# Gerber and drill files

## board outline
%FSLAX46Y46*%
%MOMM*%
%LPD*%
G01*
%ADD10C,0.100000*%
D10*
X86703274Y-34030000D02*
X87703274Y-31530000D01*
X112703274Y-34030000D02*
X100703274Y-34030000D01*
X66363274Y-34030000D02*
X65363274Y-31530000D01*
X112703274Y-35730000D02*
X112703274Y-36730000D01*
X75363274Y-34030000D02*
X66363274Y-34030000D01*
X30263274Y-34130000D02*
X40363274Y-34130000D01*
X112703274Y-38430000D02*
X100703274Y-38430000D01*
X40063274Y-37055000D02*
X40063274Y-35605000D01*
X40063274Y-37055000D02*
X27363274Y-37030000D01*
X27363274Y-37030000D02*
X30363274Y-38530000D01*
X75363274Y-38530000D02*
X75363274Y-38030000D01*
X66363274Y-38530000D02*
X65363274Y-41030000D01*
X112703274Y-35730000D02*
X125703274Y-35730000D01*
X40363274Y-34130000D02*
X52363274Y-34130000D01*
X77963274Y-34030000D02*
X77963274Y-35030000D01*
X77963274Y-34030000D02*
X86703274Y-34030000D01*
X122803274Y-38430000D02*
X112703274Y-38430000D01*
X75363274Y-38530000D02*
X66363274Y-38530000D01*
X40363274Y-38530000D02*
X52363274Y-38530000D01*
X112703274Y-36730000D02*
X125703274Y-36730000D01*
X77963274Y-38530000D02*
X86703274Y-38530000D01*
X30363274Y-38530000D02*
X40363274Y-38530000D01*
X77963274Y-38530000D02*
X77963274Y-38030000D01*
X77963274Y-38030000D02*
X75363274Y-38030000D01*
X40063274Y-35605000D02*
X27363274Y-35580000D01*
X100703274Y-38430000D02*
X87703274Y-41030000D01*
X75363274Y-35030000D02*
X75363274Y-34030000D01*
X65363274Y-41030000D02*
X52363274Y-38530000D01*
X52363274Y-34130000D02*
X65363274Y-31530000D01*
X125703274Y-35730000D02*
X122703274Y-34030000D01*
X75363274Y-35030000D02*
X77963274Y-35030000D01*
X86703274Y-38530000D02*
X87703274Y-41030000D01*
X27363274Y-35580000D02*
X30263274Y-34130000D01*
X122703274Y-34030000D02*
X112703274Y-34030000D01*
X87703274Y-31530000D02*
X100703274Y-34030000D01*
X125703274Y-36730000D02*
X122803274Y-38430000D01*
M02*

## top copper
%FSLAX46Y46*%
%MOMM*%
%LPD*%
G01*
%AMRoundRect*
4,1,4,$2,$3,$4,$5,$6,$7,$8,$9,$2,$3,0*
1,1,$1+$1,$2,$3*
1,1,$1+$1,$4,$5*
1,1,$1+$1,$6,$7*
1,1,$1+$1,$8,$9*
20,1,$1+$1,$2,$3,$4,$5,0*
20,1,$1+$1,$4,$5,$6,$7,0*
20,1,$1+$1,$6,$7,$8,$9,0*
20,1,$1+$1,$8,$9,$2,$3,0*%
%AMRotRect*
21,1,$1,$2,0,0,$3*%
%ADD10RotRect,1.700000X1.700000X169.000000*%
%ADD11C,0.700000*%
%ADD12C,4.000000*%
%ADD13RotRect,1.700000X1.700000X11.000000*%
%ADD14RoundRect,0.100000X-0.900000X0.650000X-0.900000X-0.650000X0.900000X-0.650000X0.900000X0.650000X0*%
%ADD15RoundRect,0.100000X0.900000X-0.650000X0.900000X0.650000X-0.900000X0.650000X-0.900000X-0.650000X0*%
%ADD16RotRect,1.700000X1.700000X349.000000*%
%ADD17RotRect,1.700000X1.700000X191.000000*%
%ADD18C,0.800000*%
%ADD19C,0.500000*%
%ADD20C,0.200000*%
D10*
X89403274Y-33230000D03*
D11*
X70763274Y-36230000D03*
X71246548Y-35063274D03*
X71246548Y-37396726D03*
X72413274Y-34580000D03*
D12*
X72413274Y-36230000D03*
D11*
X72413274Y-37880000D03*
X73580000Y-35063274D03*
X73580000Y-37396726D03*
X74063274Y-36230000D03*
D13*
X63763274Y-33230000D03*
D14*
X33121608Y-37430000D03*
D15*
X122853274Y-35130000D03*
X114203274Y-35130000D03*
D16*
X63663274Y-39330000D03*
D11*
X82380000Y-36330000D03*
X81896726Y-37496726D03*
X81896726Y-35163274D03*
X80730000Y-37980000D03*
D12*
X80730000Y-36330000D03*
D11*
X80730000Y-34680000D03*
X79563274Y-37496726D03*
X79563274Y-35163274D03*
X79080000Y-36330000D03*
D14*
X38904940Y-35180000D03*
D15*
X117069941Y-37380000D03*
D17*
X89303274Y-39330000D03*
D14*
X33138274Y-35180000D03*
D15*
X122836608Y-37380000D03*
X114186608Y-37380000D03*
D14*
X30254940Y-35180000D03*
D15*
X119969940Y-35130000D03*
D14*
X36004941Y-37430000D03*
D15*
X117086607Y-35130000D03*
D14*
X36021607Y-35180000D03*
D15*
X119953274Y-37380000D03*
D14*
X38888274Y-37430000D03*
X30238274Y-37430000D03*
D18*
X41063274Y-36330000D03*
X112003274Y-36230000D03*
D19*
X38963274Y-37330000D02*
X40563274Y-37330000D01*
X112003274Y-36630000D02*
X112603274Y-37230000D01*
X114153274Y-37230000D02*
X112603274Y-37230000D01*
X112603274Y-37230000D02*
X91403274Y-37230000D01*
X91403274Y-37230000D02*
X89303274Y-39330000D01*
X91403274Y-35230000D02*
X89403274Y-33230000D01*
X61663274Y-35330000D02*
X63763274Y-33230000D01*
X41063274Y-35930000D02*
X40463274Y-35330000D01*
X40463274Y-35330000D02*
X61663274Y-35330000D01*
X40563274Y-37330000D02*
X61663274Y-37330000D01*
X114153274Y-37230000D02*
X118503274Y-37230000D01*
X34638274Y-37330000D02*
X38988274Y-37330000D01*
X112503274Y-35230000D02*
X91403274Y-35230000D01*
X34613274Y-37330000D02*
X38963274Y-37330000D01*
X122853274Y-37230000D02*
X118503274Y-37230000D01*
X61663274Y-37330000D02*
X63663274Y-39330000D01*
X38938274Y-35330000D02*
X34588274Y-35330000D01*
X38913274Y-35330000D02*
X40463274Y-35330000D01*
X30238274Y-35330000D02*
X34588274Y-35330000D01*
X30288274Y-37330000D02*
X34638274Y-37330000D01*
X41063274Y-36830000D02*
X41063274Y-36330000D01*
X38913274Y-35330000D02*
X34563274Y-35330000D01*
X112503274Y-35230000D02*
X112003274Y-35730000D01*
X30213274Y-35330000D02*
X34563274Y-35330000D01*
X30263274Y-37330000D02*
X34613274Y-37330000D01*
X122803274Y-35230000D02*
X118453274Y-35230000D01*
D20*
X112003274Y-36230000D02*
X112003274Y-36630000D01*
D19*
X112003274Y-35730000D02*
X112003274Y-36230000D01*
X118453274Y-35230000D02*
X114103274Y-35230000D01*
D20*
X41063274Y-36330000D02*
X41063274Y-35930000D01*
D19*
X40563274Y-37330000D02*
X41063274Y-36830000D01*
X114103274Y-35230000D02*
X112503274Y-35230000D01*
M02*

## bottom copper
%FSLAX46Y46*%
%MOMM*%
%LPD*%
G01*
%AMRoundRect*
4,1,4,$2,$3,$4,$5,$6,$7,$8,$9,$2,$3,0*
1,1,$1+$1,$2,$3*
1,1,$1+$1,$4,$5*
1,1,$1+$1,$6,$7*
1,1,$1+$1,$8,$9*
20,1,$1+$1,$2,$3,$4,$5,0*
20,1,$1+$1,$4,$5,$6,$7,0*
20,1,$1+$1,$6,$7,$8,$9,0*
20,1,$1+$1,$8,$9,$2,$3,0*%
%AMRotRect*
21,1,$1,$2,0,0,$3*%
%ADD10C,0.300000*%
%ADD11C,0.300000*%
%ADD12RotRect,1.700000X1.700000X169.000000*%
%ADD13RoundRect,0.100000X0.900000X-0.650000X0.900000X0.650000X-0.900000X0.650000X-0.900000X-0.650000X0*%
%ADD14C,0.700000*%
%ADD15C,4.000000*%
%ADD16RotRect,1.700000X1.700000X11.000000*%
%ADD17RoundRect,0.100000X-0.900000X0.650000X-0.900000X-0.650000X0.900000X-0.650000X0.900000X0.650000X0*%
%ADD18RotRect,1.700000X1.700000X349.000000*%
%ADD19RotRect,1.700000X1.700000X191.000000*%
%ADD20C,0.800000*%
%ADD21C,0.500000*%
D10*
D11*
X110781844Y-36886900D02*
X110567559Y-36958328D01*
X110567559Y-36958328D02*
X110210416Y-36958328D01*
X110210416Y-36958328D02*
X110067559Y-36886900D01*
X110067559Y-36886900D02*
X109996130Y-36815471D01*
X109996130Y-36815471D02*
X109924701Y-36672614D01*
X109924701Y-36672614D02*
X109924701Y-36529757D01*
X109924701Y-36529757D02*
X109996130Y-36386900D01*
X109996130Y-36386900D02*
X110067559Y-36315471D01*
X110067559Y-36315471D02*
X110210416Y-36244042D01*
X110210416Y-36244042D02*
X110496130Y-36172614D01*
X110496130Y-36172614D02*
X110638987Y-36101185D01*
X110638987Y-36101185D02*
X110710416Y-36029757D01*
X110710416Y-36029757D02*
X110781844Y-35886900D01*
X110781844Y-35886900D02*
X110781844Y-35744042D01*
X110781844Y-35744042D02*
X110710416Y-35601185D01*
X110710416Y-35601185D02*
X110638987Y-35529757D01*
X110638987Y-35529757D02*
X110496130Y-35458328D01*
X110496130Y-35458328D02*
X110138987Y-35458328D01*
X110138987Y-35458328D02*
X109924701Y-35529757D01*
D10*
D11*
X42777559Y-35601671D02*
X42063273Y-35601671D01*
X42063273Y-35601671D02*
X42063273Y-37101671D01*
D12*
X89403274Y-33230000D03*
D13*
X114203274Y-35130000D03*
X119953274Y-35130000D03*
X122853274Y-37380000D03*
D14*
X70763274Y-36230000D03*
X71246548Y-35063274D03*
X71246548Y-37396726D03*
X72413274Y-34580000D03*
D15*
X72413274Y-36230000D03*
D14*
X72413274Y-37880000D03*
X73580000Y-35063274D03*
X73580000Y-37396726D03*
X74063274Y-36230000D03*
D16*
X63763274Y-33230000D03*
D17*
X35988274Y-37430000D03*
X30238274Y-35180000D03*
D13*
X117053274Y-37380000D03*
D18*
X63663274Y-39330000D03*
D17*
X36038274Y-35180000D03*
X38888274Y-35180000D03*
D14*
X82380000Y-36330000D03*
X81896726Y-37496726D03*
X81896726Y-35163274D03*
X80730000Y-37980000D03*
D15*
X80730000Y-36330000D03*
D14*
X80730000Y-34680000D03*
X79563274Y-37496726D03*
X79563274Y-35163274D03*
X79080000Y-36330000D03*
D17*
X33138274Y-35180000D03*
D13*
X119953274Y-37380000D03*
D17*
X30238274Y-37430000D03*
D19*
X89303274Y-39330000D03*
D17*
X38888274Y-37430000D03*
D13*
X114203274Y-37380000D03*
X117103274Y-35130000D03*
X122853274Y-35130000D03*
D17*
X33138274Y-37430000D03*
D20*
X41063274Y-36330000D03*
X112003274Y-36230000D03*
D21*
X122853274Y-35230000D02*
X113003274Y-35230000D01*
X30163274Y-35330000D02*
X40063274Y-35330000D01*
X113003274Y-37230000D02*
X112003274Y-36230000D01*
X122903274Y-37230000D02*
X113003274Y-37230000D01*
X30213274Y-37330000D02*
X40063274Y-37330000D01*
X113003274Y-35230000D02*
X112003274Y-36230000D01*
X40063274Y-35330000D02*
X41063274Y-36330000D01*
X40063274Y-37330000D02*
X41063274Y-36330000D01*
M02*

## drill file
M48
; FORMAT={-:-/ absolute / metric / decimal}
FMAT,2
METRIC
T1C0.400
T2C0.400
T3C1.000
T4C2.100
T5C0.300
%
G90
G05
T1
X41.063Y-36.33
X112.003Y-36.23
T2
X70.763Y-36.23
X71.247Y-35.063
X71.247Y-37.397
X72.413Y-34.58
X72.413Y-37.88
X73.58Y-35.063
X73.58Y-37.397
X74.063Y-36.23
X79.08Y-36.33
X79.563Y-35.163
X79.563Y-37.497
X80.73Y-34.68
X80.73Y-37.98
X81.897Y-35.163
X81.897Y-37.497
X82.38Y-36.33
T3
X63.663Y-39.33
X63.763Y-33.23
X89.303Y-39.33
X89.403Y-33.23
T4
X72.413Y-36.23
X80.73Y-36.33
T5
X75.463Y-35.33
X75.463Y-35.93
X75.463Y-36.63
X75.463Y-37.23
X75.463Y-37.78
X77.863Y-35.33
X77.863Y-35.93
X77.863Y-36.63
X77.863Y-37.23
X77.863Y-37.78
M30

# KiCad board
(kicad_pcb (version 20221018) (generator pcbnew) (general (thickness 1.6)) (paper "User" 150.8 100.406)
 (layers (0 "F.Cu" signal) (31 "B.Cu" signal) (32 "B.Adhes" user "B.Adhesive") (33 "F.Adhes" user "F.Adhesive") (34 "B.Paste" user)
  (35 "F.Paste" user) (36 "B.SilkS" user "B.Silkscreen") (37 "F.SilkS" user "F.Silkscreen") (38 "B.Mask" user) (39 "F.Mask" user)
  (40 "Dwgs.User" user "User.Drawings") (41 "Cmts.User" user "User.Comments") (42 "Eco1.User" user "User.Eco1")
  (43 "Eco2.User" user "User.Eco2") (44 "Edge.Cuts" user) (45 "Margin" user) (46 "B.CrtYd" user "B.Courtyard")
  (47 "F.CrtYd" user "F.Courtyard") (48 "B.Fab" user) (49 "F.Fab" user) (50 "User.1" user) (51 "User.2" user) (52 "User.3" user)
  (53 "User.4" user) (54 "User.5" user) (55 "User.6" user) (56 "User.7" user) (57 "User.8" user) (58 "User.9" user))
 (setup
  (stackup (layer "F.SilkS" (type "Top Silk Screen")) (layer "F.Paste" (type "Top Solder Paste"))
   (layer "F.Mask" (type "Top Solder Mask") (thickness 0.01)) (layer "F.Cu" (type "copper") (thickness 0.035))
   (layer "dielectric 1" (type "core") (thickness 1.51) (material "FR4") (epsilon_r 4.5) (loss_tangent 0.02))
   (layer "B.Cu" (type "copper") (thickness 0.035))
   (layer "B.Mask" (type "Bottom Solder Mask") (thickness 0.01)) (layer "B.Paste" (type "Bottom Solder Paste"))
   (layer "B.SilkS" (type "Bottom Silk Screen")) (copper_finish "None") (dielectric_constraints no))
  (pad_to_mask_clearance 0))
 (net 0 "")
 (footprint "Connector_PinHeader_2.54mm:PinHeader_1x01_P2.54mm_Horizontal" (layer "F.Cu") (at 89.403274 33.23 169)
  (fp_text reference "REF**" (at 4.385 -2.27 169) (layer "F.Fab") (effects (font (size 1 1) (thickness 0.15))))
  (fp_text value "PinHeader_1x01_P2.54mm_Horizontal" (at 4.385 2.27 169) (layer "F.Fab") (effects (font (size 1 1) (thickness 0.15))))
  (pad "1" thru_hole rect (at 0 0 169) (size 1.7 1.7) (drill 1) (layers "F&B.Cu" "*.Mask")))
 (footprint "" (layer "F.Cu") (at 114.203274 35.13)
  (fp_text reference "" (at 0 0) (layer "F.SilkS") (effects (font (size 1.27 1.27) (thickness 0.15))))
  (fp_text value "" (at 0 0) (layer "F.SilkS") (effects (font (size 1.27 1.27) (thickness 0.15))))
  (pad "2" smd roundrect (at 0 0 90) (size 1.5 2) (layers "B.Cu" "B.Paste" "B.Mask") (roundrect_rratio 0.06666666667)))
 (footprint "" (layer "F.Cu") (at 119.953274 35.13)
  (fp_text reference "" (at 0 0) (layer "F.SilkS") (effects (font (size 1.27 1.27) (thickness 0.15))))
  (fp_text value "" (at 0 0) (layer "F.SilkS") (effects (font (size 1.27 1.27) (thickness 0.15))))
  (pad "2" smd roundrect (at 0 0 90) (size 1.5 2) (layers "B.Cu" "B.Paste" "B.Mask") (roundrect_rratio 0.06666666667)))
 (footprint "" (layer "F.Cu") (at 122.853274 37.38)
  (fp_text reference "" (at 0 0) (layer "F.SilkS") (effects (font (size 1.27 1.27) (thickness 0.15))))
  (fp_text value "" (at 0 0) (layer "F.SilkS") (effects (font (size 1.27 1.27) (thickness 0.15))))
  (pad "2" smd roundrect (at 0 0 90) (size 1.5 2) (layers "B.Cu" "B.Paste" "B.Mask") (roundrect_rratio 0.06666666667)))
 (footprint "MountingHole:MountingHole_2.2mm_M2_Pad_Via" (layer "F.Cu") (at 72.413274 36.23)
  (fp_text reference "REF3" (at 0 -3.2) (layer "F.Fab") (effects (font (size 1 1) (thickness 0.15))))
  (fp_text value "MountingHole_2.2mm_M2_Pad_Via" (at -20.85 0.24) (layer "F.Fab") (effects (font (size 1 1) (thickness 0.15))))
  (pad "1" thru_hole circle (at -1.65 0) (size 0.7 0.7) (drill 0.4) (layers "F&B.Cu" "*.Mask"))
  (pad "1" thru_hole circle (at -1.166726 -1.166726) (size 0.7 0.7) (drill 0.4) (layers "F&B.Cu" "*.Mask"))
  (pad "1" thru_hole circle (at -1.166726 1.166726) (size 0.7 0.7) (drill 0.4) (layers "F&B.Cu" "*.Mask"))
  (pad "1" thru_hole circle (at 0 -1.65) (size 0.7 0.7) (drill 0.4) (layers "F&B.Cu" "*.Mask"))
  (pad "1" thru_hole circle (at 0 0) (size 4 4) (drill 2.1) (layers "F&B.Cu" "*.Mask"))
  (pad "1" thru_hole circle (at 0 1.65) (size 0.7 0.7) (drill 0.4) (layers "F&B.Cu" "*.Mask"))
  (pad "1" thru_hole circle (at 1.166726 -1.166726) (size 0.7 0.7) (drill 0.4) (layers "F&B.Cu" "*.Mask"))
  (pad "1" thru_hole circle (at 1.166726 1.166726) (size 0.7 0.7) (drill 0.4) (layers "F&B.Cu" "*.Mask"))
  (pad "1" thru_hole circle (at 1.65 0) (size 0.7 0.7) (drill 0.4) (layers "F&B.Cu" "*.Mask")))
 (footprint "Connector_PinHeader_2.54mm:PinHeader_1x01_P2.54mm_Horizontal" (layer "F.Cu") (at 63.763274 33.23 11)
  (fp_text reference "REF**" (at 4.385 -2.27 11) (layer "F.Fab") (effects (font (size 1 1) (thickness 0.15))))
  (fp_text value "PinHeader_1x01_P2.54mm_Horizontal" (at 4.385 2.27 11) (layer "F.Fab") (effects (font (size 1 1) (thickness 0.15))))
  (pad "1" thru_hole rect (at 0 0 11) (size 1.7 1.7) (drill 1) (layers "F&B.Cu" "*.Mask")))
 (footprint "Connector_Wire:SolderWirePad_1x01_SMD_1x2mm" (layer "F.Cu") (at 33.121608 37.43 -90)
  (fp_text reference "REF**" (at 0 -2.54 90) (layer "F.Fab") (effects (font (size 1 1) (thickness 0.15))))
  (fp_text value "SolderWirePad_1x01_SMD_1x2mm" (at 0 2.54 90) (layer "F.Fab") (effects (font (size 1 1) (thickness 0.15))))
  (pad "1" smd roundrect (at 0 0 270) (size 1.5 2) (layers "F.Cu" "F.Paste" "F.Mask") (roundrect_rratio 0.06666666667)))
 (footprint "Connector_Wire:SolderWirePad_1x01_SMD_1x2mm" (layer "F.Cu") (at 122.853274 35.13 90)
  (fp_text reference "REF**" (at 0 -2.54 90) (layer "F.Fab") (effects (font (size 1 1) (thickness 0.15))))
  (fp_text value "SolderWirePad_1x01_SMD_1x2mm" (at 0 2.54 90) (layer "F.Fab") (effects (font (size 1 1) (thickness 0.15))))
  (pad "1" smd roundrect (at 0 0 90) (size 1.5 2) (layers "F.Cu" "F.Paste" "F.Mask") (roundrect_rratio 0.06666666667)))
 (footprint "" (layer "F.Cu") (at 35.988274 37.43 180)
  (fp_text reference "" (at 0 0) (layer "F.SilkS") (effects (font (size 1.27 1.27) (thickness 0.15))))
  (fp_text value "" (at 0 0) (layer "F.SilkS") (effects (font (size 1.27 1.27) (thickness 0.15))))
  (pad "2" smd roundrect (at 0 0 270) (size 1.5 2) (layers "B.Cu" "B.Paste" "B.Mask") (roundrect_rratio 0.06666666667)))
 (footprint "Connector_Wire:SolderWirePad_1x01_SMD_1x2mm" (layer "F.Cu") (at 114.203274 35.13 90)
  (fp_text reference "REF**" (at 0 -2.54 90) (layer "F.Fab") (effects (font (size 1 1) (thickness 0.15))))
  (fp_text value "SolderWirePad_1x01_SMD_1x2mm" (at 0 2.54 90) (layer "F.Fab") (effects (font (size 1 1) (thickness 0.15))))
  (pad "1" smd roundrect (at 0 0 90) (size 1.5 2) (layers "F.Cu" "F.Paste" "F.Mask") (roundrect_rratio 0.06666666667)))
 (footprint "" (layer "F.Cu") (at 30.238274 35.18 180)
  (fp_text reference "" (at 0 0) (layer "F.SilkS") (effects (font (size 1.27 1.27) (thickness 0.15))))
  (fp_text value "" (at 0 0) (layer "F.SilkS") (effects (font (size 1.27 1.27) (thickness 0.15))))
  (pad "2" smd roundrect (at 0 0 270) (size 1.5 2) (layers "B.Cu" "B.Paste" "B.Mask") (roundrect_rratio 0.06666666667)))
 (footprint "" (layer "F.Cu") (at 117.053274 37.38)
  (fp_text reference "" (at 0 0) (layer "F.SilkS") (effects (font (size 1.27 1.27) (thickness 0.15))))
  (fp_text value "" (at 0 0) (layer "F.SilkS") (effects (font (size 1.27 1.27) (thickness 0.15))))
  (pad "2" smd roundrect (at 0 0 90) (size 1.5 2) (layers "B.Cu" "B.Paste" "B.Mask") (roundrect_rratio 0.06666666667)))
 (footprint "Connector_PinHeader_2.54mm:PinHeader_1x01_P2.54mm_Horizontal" (layer "F.Cu") (at 63.663274 39.33 -11)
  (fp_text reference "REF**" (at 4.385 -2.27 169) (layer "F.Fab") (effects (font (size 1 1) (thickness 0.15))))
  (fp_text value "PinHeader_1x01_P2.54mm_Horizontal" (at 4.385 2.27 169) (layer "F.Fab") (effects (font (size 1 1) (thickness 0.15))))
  (pad "1" thru_hole rect (at 0 0 349) (size 1.7 1.7) (drill 1) (layers "F&B.Cu" "*.Mask")))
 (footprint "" (layer "F.Cu") (at 36.038274 35.18 180)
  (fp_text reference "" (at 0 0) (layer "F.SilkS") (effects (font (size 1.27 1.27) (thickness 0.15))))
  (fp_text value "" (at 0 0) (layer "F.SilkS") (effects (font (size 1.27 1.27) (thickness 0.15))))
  (pad "2" smd roundrect (at 0 0 270) (size 1.5 2) (layers "B.Cu" "B.Paste" "B.Mask") (roundrect_rratio 0.06666666667)))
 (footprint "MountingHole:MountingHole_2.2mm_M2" (layer "F.Cu") (at 75.463274 36.63)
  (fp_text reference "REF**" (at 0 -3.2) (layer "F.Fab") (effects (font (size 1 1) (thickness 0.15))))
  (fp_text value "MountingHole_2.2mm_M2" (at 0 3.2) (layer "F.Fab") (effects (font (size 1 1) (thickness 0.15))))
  (pad "" np_thru_hole circle (at 0 0) (size 0.3 0.3) (drill 0.3) (layers "F&B.Cu" "*.Mask")))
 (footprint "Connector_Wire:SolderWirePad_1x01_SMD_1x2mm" (layer "F.Cu") (at 38.888274 35.18 -90)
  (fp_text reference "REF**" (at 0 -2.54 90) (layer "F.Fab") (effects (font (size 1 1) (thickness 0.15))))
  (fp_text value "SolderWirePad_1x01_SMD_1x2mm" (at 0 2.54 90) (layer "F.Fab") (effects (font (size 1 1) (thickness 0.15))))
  (pad "2" smd roundrect (at 0 0 270) (size 1.5 2) (layers "B.Cu" "B.Paste" "B.Mask") (roundrect_rratio 0.06666666667)))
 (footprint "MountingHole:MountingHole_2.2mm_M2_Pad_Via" (layer "F.Cu") (at 80.73 36.33 180)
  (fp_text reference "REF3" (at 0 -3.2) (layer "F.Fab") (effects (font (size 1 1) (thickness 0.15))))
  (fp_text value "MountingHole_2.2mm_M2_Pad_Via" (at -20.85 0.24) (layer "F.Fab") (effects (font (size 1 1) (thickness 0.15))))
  (pad "1" thru_hole circle (at -1.65 0 180) (size 0.7 0.7) (drill 0.4) (layers "F&B.Cu" "*.Mask"))
  (pad "1" thru_hole circle (at -1.166726 -1.166726 180) (size 0.7 0.7) (drill 0.4) (layers "F&B.Cu" "*.Mask"))
  (pad "1" thru_hole circle (at -1.166726 1.166726 180) (size 0.7 0.7) (drill 0.4) (layers "F&B.Cu" "*.Mask"))
  (pad "1" thru_hole circle (at 0 -1.65 180) (size 0.7 0.7) (drill 0.4) (layers "F&B.Cu" "*.Mask"))
  (pad "1" thru_hole circle (at 0 0 180) (size 4 4) (drill 2.1) (layers "*.Cu" "*.Mask"))
  (pad "1" thru_hole circle (at 0 1.65 180) (size 0.7 0.7) (drill 0.4) (layers "F&B.Cu" "*.Mask"))
  (pad "1" thru_hole circle (at 1.166726 -1.166726 180) (size 0.7 0.7) (drill 0.4) (layers "F&B.Cu" "*.Mask"))
  (pad "1" thru_hole circle (at 1.166726 1.166726 180) (size 0.7 0.7) (drill 0.4) (layers "F&B.Cu" "*.Mask"))
  (pad "1" thru_hole circle (at 1.65 0 180) (size 0.7 0.7) (drill 0.4) (layers "F&B.Cu" "*.Mask")))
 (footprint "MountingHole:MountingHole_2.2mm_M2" (layer "F.Cu") (at 75.463274 37.78)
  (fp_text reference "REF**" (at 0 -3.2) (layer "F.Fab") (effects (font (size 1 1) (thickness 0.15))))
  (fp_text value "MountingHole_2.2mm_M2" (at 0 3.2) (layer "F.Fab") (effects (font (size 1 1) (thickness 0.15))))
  (pad "" np_thru_hole circle (at 0 0) (size 0.3 0.3) (drill 0.3) (layers "F&B.Cu" "*.Mask")))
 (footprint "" (layer "F.Cu") (at 33.138274 35.18 180)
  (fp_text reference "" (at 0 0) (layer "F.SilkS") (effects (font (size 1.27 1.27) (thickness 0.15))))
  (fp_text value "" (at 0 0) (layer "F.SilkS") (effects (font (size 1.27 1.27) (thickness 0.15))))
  (pad "2" smd roundrect (at 0 0 270) (size 1.5 2) (layers "B.Cu" "B.Paste" "B.Mask") (roundrect_rratio 0.06666666667)))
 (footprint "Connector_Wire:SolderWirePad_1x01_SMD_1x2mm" (layer "F.Cu") (at 38.90494 35.18 -90)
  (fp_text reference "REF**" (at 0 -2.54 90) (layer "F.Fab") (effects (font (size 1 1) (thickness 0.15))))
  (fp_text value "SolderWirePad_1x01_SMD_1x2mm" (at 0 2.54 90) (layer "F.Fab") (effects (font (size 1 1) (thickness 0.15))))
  (pad "1" smd roundrect (at 0 0 270) (size 1.5 2) (layers "F.Cu" "F.Paste" "F.Mask") (roundrect_rratio 0.06666666667)))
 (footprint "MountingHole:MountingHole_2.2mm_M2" (layer "F.Cu") (at 77.863274 36.63)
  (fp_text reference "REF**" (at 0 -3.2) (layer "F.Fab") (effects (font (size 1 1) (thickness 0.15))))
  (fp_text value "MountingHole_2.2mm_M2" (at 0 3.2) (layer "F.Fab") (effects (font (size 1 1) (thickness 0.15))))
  (pad "" np_thru_hole circle (at 0 0) (size 0.3 0.3) (drill 0.3) (layers "F&B.Cu" "*.Mask")))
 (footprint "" (layer "F.Cu") (at 119.953274 37.38)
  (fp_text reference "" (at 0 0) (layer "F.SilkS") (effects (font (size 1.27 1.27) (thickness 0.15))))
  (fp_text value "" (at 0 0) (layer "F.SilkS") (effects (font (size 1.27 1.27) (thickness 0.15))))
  (pad "2" smd roundrect (at 0 0 90) (size 1.5 2) (layers "B.Cu" "B.Paste" "B.Mask") (roundrect_rratio 0.06666666667)))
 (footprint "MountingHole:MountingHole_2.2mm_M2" (layer "F.Cu") (at 77.863274 35.93)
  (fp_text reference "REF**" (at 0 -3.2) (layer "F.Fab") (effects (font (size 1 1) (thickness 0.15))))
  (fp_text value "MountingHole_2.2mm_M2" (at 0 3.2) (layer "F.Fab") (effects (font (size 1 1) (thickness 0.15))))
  (pad "" np_thru_hole circle (at 0 0) (size 0.3 0.3) (drill 0.3) (layers "F&B.Cu" "*.Mask")))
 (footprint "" (layer "F.Cu") (at 30.238274 37.43 180)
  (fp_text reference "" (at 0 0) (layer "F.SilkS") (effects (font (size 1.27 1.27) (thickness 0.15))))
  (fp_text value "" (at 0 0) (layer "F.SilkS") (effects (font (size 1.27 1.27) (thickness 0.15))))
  (pad "2" smd roundrect (at 0 0 270) (size 1.5 2) (layers "B.Cu" "B.Paste" "B.Mask") (roundrect_rratio 0.06666666667)))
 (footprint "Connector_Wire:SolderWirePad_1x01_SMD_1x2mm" (layer "F.Cu") (at 117.069941 37.38 90)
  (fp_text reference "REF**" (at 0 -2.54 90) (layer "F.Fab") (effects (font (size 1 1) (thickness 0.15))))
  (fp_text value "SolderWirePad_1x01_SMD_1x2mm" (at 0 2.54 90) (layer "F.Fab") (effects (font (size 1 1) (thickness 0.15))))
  (pad "1" smd roundrect (at 0 0 90) (size 1.5 2) (layers "F.Cu" "F.Paste" "F.Mask") (roundrect_rratio 0.06666666667)))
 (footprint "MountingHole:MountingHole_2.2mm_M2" (layer "F.Cu") (at 75.463274 35.93)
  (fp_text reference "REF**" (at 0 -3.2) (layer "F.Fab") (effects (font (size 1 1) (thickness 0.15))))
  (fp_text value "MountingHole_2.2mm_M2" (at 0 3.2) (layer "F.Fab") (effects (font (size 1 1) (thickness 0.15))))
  (pad "" np_thru_hole circle (at 0 0) (size 0.3 0.3) (drill 0.3) (layers "F&B.Cu" "*.Mask")))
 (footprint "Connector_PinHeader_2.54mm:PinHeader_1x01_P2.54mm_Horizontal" (layer "F.Cu") (at 89.303274 39.33 -169)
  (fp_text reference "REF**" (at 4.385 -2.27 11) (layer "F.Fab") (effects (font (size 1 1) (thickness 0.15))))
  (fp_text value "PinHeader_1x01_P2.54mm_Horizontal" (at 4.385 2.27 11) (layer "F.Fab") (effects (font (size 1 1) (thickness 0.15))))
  (pad "1" thru_hole rect (at 0 0 191) (size 1.7 1.7) (drill 1) (layers "F&B.Cu" "*.Mask")))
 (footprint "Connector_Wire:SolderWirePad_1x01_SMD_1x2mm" (layer "F.Cu") (at 33.138274 35.18 -90)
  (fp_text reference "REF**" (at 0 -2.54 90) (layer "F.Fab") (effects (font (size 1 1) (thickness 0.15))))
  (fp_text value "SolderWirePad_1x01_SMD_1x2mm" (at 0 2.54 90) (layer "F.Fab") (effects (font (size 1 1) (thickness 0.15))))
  (pad "1" smd roundrect (at 0 0 270) (size 1.5 2) (layers "F.Cu" "F.Paste" "F.Mask") (roundrect_rratio 0.06666666667)))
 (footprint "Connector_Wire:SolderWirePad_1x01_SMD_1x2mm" (layer "F.Cu") (at 122.836608 37.38 90)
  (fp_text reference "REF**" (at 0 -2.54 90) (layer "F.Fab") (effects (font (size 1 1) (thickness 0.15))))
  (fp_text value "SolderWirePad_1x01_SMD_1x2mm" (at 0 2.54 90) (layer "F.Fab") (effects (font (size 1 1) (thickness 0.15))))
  (pad "1" smd roundrect (at 0 0 90) (size 1.5 2) (layers "F.Cu" "F.Paste" "F.Mask") (roundrect_rratio 0.06666666667)))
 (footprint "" (layer "F.Cu") (at 38.888274 37.43 180)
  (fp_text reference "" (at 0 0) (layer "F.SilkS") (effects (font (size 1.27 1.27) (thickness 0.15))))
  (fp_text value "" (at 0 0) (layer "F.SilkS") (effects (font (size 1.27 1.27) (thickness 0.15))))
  (pad "2" smd roundrect (at 0 0 270) (size 1.5 2) (layers "B.Cu" "B.Paste" "B.Mask") (roundrect_rratio 0.06666666667)))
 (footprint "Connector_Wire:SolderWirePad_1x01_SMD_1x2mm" (layer "F.Cu") (at 114.186608 37.38 90)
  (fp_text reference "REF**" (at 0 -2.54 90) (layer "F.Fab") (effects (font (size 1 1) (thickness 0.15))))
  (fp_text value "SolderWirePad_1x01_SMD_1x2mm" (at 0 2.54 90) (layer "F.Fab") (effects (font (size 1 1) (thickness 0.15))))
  (pad "1" smd roundrect (at 0 0 90) (size 1.5 2) (layers "F.Cu" "F.Paste" "F.Mask") (roundrect_rratio 0.06666666667)))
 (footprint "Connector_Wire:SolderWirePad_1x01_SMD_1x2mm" (layer "F.Cu") (at 30.25494 35.18 -90)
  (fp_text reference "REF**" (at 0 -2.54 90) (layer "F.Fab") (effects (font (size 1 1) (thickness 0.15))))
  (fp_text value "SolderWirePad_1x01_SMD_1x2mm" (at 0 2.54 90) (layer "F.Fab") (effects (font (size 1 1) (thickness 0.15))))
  (pad "1" smd roundrect (at 0 0 270) (size 1.5 2) (layers "F.Cu" "F.Paste" "F.Mask") (roundrect_rratio 0.06666666667)))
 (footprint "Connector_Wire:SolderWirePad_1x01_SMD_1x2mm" (layer "F.Cu") (at 119.96994 35.13 90)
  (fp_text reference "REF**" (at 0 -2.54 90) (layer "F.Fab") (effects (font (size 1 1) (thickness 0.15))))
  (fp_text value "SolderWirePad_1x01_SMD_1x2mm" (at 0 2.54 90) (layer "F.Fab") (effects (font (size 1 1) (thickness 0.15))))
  (pad "1" smd roundrect (at 0 0 90) (size 1.5 2) (layers "F.Cu" "F.Paste" "F.Mask") (roundrect_rratio 0.06666666667)))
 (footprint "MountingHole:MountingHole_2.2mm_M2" (layer "F.Cu") (at 77.863274 37.23)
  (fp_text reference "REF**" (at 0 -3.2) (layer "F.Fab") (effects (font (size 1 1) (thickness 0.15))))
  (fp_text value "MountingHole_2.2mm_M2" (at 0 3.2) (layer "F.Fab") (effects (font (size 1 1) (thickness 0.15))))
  (pad "" np_thru_hole circle (at 0 0) (size 0.3 0.3) (drill 0.3) (layers "F&B.Cu" "*.Mask")))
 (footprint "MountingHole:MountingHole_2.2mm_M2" (layer "F.Cu") (at 75.463274 35.33)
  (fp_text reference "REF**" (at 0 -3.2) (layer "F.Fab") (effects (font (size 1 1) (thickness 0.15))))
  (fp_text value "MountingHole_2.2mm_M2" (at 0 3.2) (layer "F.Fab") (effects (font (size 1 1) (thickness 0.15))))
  (pad "" np_thru_hole circle (at 0 0) (size 0.3 0.3) (drill 0.3) (layers "F&B.Cu" "*.Mask")))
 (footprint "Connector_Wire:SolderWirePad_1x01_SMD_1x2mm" (layer "F.Cu") (at 36.004941 37.43 -90)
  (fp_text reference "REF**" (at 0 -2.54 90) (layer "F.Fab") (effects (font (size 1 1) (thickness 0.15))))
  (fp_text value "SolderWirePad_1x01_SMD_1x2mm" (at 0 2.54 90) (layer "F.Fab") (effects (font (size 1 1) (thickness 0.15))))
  (pad "1" smd roundrect (at 0 0 270) (size 1.5 2) (layers "F.Cu" "F.Paste" "F.Mask") (roundrect_rratio 0.06666666667)))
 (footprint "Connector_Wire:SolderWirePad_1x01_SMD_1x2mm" (layer "F.Cu") (at 114.203274 37.38 90)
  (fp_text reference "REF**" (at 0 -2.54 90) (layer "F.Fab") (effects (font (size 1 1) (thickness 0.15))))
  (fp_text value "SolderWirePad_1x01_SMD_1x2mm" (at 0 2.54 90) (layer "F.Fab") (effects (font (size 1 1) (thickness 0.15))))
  (pad "2" smd roundrect (at 0 0 90) (size 1.5 2) (layers "B.Cu" "B.Paste" "B.Mask") (roundrect_rratio 0.06666666667)))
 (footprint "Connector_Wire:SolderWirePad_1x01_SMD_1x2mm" (layer "F.Cu") (at 117.086607 35.13 90)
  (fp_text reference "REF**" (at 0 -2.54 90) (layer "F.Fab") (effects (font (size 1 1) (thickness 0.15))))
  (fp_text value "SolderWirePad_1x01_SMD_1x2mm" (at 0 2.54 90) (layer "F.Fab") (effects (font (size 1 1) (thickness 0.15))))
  (pad "1" smd roundrect (at 0 0 90) (size 1.5 2) (layers "F.Cu" "F.Paste" "F.Mask") (roundrect_rratio 0.06666666667)))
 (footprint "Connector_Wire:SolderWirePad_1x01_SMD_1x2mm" (layer "F.Cu") (at 36.021607 35.18 -90)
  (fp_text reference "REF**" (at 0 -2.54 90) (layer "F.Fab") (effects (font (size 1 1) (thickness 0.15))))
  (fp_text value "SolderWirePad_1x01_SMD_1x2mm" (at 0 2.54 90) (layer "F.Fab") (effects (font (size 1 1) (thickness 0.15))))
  (pad "1" smd roundrect (at 0 0 270) (size 1.5 2) (layers "F.Cu" "F.Paste" "F.Mask") (roundrect_rratio 0.06666666667)))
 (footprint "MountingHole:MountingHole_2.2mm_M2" (layer "F.Cu") (at 75.463274 37.23)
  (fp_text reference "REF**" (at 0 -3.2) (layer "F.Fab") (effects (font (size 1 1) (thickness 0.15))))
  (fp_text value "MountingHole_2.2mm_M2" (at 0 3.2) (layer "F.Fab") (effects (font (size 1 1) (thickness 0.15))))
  (pad "" np_thru_hole circle (at 0 0) (size 0.3 0.3) (drill 0.3) (layers "F&B.Cu" "*.Mask")))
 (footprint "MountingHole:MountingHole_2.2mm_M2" (layer "F.Cu") (at 77.863274 35.33)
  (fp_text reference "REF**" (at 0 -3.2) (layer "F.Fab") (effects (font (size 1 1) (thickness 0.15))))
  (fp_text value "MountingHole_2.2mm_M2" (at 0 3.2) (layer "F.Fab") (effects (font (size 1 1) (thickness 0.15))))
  (pad "" np_thru_hole circle (at 0 0) (size 0.3 0.3) (drill 0.3) (layers "F&B.Cu" "*.Mask")))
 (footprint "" (layer "F.Cu") (at 117.103274 35.13)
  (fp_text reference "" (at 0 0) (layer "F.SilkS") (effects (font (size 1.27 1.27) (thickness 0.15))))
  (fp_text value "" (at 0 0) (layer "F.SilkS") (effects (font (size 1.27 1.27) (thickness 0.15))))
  (pad "2" smd roundrect (at 0 0 90) (size 1.5 2) (layers "B.Cu" "B.Paste" "B.Mask") (roundrect_rratio 0.06666666667)))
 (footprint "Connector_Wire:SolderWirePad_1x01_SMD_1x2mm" (layer "F.Cu") (at 119.953274 37.38 90)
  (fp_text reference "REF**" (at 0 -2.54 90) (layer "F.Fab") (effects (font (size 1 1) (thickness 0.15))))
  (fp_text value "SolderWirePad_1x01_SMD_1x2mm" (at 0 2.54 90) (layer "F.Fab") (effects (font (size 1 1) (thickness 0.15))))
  (pad "1" smd roundrect (at 0 0 90) (size 1.5 2) (layers "F.Cu" "F.Paste" "F.Mask") (roundrect_rratio 0.06666666667)))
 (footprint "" (layer "F.Cu") (at 122.853274 35.13)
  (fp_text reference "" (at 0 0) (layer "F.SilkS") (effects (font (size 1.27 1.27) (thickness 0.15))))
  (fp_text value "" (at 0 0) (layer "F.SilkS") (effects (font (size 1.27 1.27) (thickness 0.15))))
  (pad "2" smd roundrect (at 0 0 90) (size 1.5 2) (layers "B.Cu" "B.Paste" "B.Mask") (roundrect_rratio 0.06666666667)))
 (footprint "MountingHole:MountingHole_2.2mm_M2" (layer "F.Cu") (at 77.863274 37.78)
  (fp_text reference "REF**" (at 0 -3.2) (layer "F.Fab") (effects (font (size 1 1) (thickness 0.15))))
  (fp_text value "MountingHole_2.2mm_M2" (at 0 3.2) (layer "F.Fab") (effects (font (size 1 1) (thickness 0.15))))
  (pad "" np_thru_hole circle (at 0 0) (size 0.3 0.3) (drill 0.3) (layers "F&B.Cu" "*.Mask")))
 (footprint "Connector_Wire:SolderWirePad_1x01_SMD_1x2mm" (layer "F.Cu") (at 38.888274 37.43 -90)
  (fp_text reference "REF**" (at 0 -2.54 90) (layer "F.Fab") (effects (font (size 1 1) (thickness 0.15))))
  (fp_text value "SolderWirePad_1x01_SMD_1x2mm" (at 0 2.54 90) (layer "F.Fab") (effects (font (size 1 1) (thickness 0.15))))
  (pad "1" smd roundrect (at 0 0 270) (size 1.5 2) (layers "F.Cu" "F.Paste" "F.Mask") (roundrect_rratio 0.06666666667)))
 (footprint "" (layer "F.Cu") (at 33.138274 37.43 180)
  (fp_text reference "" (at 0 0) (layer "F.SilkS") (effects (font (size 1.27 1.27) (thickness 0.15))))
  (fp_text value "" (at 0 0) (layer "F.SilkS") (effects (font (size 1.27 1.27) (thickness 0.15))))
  (pad "2" smd roundrect (at 0 0 270) (size 1.5 2) (layers "B.Cu" "B.Paste" "B.Mask") (roundrect_rratio 0.06666666667)))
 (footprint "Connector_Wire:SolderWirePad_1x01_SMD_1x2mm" (layer "F.Cu") (at 30.238274 37.43 -90)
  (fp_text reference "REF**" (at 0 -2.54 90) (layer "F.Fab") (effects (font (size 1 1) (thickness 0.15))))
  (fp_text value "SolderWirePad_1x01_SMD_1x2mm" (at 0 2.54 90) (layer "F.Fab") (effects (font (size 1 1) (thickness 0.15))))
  (pad "1" smd roundrect (at 0 0 270) (size 1.5 2) (layers "F.Cu" "F.Paste" "F.Mask") (roundrect_rratio 0.06666666667)))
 (gr_line (start 86.703274 34.03) (end 87.703274 31.53) (stroke (width 0.1) (type solid)) (layer "Edge.Cuts"))
 (gr_line (start 112.703274 34.03) (end 100.703274 34.03) (stroke (width 0.1) (type solid)) (layer "Edge.Cuts"))
 (gr_line (start 66.363274 34.03) (end 65.363274 31.53) (stroke (width 0.1) (type solid)) (layer "Edge.Cuts"))
 (gr_line (start 112.703274 35.73) (end 112.703274 36.73) (stroke (width 0.1) (type solid)) (layer "Edge.Cuts"))
 (gr_line (start 75.363274 34.03) (end 66.363274 34.03) (stroke (width 0.1) (type solid)) (layer "Edge.Cuts"))
 (gr_line (start 30.263274 34.13) (end 40.363274 34.13) (stroke (width 0.1) (type solid)) (layer "Edge.Cuts"))
 (gr_line (start 112.703274 38.43) (end 100.703274 38.43) (stroke (width 0.1) (type solid)) (layer "Edge.Cuts"))
 (gr_line (start 40.063274 37.055) (end 40.063274 35.605) (stroke (width 0.1) (type solid)) (layer "Edge.Cuts"))
 (gr_line (start 40.063274 37.055) (end 27.363274 37.03) (stroke (width 0.1) (type solid)) (layer "Edge.Cuts"))
 (gr_line (start 27.363274 37.03) (end 30.363274 38.53) (stroke (width 0.1) (type solid)) (layer "Edge.Cuts"))
 (gr_line (start 75.363274 38.53) (end 75.363274 38.03) (stroke (width 0.1) (type solid)) (layer "Edge.Cuts"))
 (gr_line (start 66.363274 38.53) (end 65.363274 41.03) (stroke (width 0.1) (type solid)) (layer "Edge.Cuts"))
 (gr_line (start 112.703274 35.73) (end 125.703274 35.73) (stroke (width 0.1) (type solid)) (layer "Edge.Cuts"))
 (gr_line (start 40.363274 34.13) (end 52.363274 34.13) (stroke (width 0.1) (type solid)) (layer "Edge.Cuts"))
 (gr_line (start 77.963274 34.03) (end 77.963274 35.03) (stroke (width 0.1) (type solid)) (layer "Edge.Cuts"))
 (gr_line (start 77.963274 34.03) (end 86.703274 34.03) (stroke (width 0.1) (type solid)) (layer "Edge.Cuts"))
 (gr_line (start 122.803274 38.43) (end 112.703274 38.43) (stroke (width 0.1) (type solid)) (layer "Edge.Cuts"))
 (gr_line (start 75.363274 38.53) (end 66.363274 38.53) (stroke (width 0.1) (type solid)) (layer "Edge.Cuts"))
 (gr_line (start 40.363274 38.53) (end 52.363274 38.53) (stroke (width 0.1) (type solid)) (layer "Edge.Cuts"))
 (gr_line (start 112.703274 36.73) (end 125.703274 36.73) (stroke (width 0.1) (type solid)) (layer "Edge.Cuts"))
 (gr_line (start 77.963274 38.53) (end 86.703274 38.53) (stroke (width 0.1) (type solid)) (layer "Edge.Cuts"))
 (gr_line (start 30.363274 38.53) (end 40.363274 38.53) (stroke (width 0.1) (type solid)) (layer "Edge.Cuts"))
 (gr_line (start 77.963274 38.53) (end 77.963274 38.03) (stroke (width 0.1) (type solid)) (layer "Edge.Cuts"))
 (gr_line (start 77.963274 38.03) (end 75.363274 38.03) (stroke (width 0.1) (type solid)) (layer "Edge.Cuts"))
 (gr_line (start 40.063274 35.605) (end 27.363274 35.58) (stroke (width 0.1) (type solid)) (layer "Edge.Cuts"))
 (gr_line (start 100.703274 38.43) (end 87.703274 41.03) (stroke (width 0.1) (type solid)) (layer "Edge.Cuts"))
 (gr_line (start 75.363274 35.03) (end 75.363274 34.03) (stroke (width 0.1) (type solid)) (layer "Edge.Cuts"))
 (gr_line (start 65.363274 41.03) (end 52.363274 38.53) (stroke (width 0.1) (type solid)) (layer "Edge.Cuts"))
 (gr_line (start 52.363274 34.13) (end 65.363274 31.53) (stroke (width 0.1) (type solid)) (layer "Edge.Cuts"))
 (gr_line (start 125.703274 35.73) (end 122.703274 34.03) (stroke (width 0.1) (type solid)) (layer "Edge.Cuts"))
 (gr_line (start 75.363274 35.03) (end 77.963274 35.03) (stroke (width 0.1) (type solid)) (layer "Edge.Cuts"))
 (gr_line (start 86.703274 38.53) (end 87.703274 41.03) (stroke (width 0.1) (type solid)) (layer "Edge.Cuts"))
 (gr_line (start 27.363274 35.58) (end 30.263274 34.13) (stroke (width 0.1) (type solid)) (layer "Edge.Cuts"))
 (gr_line (start 122.703274 34.03) (end 112.703274 34.03) (stroke (width 0.1) (type solid)) (layer "Edge.Cuts"))
 (gr_line (start 87.703274 31.53) (end 100.703274 34.03) (stroke (width 0.1) (type solid)) (layer "Edge.Cuts"))
 (gr_line (start 125.703274 36.73) (end 122.803274 38.43) (stroke (width 0.1) (type solid)) (layer "Edge.Cuts"))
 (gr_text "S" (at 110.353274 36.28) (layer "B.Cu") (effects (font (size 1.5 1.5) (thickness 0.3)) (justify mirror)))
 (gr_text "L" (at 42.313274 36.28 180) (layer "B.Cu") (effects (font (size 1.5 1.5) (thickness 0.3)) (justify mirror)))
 (segment (start 38.963274 37.33) (end 40.563274 37.33) (width 0.5) (layer "F.Cu") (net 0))
 (segment (start 112.003274 36.63) (end 112.603274 37.23) (width 0.5) (layer "F.Cu") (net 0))
 (segment (start 114.153274 37.23) (end 112.603274 37.23) (width 0.5) (layer "F.Cu") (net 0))
 (segment (start 112.603274 37.23) (end 91.403274 37.23) (width 0.5) (layer "F.Cu") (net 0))
 (segment (start 91.403274 37.23) (end 89.303274 39.33) (width 0.5) (layer "F.Cu") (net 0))
 (segment (start 91.403274 35.23) (end 89.403274 33.23) (width 0.5) (layer "F.Cu") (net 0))
 (segment (start 61.663274 35.33) (end 63.763274 33.23) (width 0.5) (layer "F.Cu") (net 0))
 (segment (start 41.063274 35.93) (end 40.463274 35.33) (width 0.5) (layer "F.Cu") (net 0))
 (segment (start 40.463274 35.33) (end 61.663274 35.33) (width 0.5) (layer "F.Cu") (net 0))
 (segment (start 40.563274 37.33) (end 61.663274 37.33) (width 0.5) (layer "F.Cu") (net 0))
 (segment (start 114.153274 37.23) (end 118.503274 37.23) (width 0.5) (layer "F.Cu") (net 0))
 (segment (start 34.638274 37.33) (end 38.988274 37.33) (width 0.5) (layer "F.Cu") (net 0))
 (segment (start 112.503274 35.23) (end 91.403274 35.23) (width 0.5) (layer "F.Cu") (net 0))
 (segment (start 34.613274 37.33) (end 38.963274 37.33) (width 0.5) (layer "F.Cu") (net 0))
 (segment (start 122.853274 37.23) (end 118.503274 37.23) (width 0.5) (layer "F.Cu") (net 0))
 (segment (start 61.663274 37.33) (end 63.663274 39.33) (width 0.5) (layer "F.Cu") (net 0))
 (segment (start 38.938274 35.33) (end 34.588274 35.33) (width 0.5) (layer "F.Cu") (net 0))
 (segment (start 38.913274 35.33) (end 40.463274 35.33) (width 0.5) (layer "F.Cu") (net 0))
 (segment (start 30.238274 35.33) (end 34.588274 35.33) (width 0.5) (layer "F.Cu") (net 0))
 (segment (start 30.288274 37.33) (end 34.638274 37.33) (width 0.5) (layer "F.Cu") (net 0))
 (segment (start 41.063274 36.83) (end 41.063274 36.33) (width 0.5) (layer "F.Cu") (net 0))
 (segment (start 38.913274 35.33) (end 34.563274 35.33) (width 0.5) (layer "F.Cu") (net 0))
 (segment (start 112.503274 35.23) (end 112.003274 35.73) (width 0.5) (layer "F.Cu") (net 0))
 (segment (start 30.213274 35.33) (end 34.563274 35.33) (width 0.5) (layer "F.Cu") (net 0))
 (segment (start 30.263274 37.33) (end 34.613274 37.33) (width 0.5) (layer "F.Cu") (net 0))
 (segment (start 122.803274 35.23) (end 118.453274 35.23) (width 0.5) (layer "F.Cu") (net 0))
 (segment (start 112.003274 36.23) (end 112.003274 36.63) (width 0.2) (layer "F.Cu") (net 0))
 (segment (start 112.003274 35.73) (end 112.003274 36.23) (width 0.5) (layer "F.Cu") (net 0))
 (segment (start 118.453274 35.23) (end 114.103274 35.23) (width 0.5) (layer "F.Cu") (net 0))
 (segment (start 41.063274 36.33) (end 41.063274 35.93) (width 0.2) (layer "F.Cu") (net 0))
 (segment (start 40.563274 37.33) (end 41.063274 36.83) (width 0.5) (layer "F.Cu") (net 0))
 (segment (start 114.103274 35.23) (end 112.503274 35.23) (width 0.5) (layer "F.Cu") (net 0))
 (via (at 41.063274 36.33) (size 0.8) (drill 0.4) (layers "F.Cu" "B.Cu") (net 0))
 (via (at 112.003274 36.23) (size 0.8) (drill 0.4) (layers "F.Cu" "B.Cu") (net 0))
 (segment (start 122.853274 35.23) (end 113.003274 35.23) (width 0.5) (layer "B.Cu") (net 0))
 (segment (start 30.163274 35.33) (end 40.063274 35.33) (width 0.5) (layer "B.Cu") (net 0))
 (segment (start 113.003274 37.23) (end 112.003274 36.23) (width 0.5) (layer "B.Cu") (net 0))
 (segment (start 122.903274 37.23) (end 113.003274 37.23) (width 0.5) (layer "B.Cu") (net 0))
 (segment (start 30.213274 37.33) (end 40.063274 37.33) (width 0.5) (layer "B.Cu") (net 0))
 (segment (start 113.003274 35.23) (end 112.003274 36.23) (width 0.5) (layer "B.Cu") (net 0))
 (segment (start 40.063274 35.33) (end 41.063274 36.33) (width 0.5) (layer "B.Cu") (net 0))
 (segment (start 40.063274 37.33) (end 41.063274 36.33) (width 0.5) (layer "B.Cu") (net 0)))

